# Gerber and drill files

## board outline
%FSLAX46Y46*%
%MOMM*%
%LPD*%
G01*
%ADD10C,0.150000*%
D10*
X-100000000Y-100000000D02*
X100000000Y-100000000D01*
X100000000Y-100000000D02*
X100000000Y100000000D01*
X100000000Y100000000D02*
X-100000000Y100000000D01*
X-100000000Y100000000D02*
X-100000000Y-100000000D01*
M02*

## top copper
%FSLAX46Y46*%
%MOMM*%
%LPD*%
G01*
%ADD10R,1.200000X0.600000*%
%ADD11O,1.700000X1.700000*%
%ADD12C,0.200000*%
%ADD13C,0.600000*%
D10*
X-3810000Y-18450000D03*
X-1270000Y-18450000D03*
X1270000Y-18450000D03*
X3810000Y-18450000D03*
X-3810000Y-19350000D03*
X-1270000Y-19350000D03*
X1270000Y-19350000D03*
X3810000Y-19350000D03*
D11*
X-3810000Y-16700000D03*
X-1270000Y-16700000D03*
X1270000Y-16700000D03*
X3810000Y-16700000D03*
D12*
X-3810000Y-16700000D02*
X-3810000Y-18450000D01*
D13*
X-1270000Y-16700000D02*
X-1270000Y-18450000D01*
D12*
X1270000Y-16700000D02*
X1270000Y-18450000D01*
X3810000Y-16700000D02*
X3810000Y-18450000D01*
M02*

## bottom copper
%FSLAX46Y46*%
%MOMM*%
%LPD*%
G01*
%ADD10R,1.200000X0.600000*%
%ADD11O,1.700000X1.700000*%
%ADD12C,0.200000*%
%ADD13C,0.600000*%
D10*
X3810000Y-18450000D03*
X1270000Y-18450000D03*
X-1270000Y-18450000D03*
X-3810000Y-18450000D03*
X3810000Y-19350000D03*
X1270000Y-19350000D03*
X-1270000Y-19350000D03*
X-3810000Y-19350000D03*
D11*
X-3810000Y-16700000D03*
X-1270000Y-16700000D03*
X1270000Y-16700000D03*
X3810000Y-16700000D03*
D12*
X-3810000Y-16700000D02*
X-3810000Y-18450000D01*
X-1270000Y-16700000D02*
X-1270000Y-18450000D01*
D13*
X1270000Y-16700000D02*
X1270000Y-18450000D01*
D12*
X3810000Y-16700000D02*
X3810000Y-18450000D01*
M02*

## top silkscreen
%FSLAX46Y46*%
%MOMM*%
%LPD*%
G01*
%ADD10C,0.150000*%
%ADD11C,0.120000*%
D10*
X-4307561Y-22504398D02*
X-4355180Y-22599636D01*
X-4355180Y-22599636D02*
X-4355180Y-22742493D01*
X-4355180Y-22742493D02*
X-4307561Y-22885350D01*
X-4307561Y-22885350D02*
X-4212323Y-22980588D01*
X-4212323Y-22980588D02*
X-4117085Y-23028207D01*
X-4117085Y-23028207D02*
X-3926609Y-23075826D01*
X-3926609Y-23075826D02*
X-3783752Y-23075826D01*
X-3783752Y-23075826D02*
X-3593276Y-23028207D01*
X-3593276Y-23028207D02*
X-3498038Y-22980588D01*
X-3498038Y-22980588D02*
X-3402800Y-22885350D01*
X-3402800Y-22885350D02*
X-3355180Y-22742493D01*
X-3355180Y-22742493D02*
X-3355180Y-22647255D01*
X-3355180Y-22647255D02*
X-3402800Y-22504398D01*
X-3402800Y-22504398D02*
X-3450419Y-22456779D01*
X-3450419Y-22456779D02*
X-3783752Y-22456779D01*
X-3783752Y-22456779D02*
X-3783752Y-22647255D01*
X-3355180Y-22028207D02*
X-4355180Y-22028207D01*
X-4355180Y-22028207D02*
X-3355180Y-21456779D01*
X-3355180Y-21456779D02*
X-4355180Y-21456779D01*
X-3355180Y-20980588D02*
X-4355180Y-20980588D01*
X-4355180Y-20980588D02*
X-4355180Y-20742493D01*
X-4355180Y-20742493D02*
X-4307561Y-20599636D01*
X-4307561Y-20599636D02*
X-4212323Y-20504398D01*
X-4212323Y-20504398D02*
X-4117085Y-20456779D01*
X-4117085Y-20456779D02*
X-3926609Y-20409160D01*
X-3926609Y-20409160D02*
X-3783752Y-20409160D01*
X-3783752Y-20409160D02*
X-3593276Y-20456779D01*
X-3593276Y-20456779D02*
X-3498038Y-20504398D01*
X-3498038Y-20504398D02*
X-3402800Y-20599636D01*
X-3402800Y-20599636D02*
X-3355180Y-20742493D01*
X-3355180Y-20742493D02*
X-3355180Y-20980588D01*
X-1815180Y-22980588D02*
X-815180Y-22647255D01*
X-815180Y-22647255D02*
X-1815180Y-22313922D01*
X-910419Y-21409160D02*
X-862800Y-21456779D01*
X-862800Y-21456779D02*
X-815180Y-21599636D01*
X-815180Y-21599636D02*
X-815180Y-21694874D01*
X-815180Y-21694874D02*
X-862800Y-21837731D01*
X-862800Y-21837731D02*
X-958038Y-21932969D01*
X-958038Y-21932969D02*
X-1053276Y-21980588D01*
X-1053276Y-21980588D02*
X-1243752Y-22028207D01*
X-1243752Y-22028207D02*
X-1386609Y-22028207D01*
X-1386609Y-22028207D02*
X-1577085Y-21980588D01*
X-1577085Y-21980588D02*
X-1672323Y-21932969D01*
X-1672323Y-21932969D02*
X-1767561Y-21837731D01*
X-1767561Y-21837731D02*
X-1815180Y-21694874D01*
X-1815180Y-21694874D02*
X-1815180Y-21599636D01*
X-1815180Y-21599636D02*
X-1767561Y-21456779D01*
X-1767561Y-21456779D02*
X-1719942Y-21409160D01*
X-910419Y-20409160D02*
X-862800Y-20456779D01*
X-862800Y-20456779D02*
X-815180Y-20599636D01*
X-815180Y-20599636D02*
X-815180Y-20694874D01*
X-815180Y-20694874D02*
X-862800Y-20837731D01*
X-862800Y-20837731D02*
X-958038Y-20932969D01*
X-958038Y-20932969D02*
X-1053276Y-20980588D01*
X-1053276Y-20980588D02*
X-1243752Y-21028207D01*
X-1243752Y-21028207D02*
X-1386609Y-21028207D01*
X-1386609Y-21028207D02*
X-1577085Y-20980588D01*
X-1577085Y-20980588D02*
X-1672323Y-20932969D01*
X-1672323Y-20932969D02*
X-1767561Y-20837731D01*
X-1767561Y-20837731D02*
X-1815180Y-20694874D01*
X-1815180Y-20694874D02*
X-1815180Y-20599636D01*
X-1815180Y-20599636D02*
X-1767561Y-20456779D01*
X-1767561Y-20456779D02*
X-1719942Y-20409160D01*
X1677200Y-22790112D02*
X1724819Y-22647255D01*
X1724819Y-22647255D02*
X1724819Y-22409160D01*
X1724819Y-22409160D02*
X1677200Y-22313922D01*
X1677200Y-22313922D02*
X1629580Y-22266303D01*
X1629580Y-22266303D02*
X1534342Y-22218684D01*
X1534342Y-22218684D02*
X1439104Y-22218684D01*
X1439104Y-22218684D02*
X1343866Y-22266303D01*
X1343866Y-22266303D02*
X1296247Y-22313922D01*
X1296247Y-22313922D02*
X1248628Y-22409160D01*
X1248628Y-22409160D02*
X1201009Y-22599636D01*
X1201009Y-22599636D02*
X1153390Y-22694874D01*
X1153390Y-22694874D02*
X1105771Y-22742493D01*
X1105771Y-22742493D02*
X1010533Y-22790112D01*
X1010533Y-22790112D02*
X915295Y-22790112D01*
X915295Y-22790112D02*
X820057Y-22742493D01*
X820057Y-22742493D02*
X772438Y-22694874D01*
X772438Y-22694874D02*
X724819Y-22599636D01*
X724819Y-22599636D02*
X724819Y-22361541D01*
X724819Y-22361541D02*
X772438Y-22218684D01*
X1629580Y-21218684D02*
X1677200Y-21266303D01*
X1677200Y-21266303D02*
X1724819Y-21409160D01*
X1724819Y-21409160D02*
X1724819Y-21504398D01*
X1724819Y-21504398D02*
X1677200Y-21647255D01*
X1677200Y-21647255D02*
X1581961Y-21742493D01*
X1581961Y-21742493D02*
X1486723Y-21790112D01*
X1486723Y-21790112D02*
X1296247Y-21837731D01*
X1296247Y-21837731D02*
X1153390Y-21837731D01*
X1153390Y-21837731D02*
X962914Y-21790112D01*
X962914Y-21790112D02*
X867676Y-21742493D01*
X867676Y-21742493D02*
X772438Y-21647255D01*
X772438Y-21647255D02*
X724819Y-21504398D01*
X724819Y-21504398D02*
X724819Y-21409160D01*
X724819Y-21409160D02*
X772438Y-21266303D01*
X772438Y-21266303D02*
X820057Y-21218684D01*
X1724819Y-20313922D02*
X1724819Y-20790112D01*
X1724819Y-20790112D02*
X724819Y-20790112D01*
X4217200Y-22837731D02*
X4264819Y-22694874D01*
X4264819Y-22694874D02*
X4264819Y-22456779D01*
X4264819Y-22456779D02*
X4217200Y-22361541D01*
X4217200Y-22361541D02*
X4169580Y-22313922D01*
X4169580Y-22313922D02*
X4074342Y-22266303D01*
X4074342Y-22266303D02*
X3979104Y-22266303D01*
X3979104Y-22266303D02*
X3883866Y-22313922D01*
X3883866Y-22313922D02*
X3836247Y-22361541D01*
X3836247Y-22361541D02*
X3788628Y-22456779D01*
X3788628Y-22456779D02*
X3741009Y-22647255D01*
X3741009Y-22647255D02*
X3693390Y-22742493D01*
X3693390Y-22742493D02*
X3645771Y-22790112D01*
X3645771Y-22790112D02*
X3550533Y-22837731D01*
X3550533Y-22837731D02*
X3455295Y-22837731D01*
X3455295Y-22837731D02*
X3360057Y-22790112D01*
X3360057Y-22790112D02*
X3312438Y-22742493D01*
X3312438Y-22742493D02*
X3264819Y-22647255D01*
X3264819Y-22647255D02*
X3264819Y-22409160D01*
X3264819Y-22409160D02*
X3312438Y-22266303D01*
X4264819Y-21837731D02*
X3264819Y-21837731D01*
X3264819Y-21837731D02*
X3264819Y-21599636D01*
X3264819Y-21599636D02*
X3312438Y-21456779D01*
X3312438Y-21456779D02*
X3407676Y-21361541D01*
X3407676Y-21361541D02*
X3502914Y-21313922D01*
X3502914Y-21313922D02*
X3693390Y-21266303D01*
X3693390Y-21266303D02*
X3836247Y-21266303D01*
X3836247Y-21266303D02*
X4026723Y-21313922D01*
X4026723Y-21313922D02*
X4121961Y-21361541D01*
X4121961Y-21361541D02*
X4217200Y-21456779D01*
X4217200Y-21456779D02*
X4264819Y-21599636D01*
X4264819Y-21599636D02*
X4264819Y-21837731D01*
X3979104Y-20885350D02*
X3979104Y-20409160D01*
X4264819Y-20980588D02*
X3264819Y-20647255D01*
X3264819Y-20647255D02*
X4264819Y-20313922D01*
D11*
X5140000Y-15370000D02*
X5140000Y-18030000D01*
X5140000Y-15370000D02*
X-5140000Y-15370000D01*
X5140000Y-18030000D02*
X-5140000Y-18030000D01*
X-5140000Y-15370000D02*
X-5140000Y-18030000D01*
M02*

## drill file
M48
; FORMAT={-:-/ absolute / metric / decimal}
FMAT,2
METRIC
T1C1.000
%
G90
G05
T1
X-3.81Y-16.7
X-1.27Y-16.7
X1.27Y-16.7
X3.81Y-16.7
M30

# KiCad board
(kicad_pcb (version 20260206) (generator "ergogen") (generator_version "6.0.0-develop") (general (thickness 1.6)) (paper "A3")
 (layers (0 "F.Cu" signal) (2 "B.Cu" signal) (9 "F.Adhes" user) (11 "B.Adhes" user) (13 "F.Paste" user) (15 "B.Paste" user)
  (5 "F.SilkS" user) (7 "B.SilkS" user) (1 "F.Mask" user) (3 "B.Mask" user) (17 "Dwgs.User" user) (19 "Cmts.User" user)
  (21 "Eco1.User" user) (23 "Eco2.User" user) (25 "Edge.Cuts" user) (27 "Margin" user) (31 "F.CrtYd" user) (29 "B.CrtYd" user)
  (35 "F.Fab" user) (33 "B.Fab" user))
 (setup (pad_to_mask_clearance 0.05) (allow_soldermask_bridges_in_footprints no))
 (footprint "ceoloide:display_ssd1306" (layer "F.Cu") (at 0 0 0)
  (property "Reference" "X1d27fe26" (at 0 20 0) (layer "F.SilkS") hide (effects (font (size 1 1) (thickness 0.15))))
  (fp_line (start 5.14 15.37) (end 5.14 18.03) (layer "F.SilkS") (stroke (width 0.12) (type solid)))
  (fp_line (start 5.14 15.37) (end -5.14 15.37) (layer "F.SilkS") (stroke (width 0.12) (type solid)))
  (fp_line (start 5.14 18.03) (end -5.14 18.03) (layer "F.SilkS") (stroke (width 0.12) (type solid)))
  (fp_line (start -5.14 15.37) (end -5.14 18.03) (layer "F.SilkS") (stroke (width 0.12) (type solid)))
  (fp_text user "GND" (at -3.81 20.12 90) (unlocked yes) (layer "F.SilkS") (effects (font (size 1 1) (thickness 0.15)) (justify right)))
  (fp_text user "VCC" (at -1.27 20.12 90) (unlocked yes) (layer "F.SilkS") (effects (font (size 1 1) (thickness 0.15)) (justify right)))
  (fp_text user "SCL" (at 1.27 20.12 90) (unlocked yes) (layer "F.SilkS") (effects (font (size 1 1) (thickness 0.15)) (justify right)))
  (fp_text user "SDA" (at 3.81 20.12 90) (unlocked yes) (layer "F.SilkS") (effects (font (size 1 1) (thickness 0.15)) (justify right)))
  (pad "14" smd rect (at -3.81 18.450000000000003 90) (size 0.6 1.2) (layers "F.Cu" "F.Paste" "F.Mask") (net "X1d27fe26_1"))
  (pad "15" smd rect (at -1.27 18.450000000000003 90) (size 0.6 1.2) (layers "F.Cu" "F.Paste" "F.Mask") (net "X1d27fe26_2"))
  (pad "16" smd rect (at 1.27 18.450000000000003 90) (size 0.6 1.2) (layers "F.Cu" "F.Paste" "F.Mask") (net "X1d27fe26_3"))
  (pad "17" smd rect (at 3.81 18.450000000000003 90) (size 0.6 1.2) (layers "F.Cu" "F.Paste" "F.Mask") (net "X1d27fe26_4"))
  (pad "10" smd rect (at -3.81 19.35 90) (size 0.6 1.2) (layers "F.Cu" "F.Paste" "F.Mask") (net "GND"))
  (pad "11" smd rect (at -1.27 19.35 90) (size 0.6 1.2) (layers "F.Cu" "F.Paste" "F.Mask") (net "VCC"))
  (pad "12" smd rect (at 1.27 19.35 90) (size 0.6 1.2) (layers "F.Cu" "F.Paste" "F.Mask") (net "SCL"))
  (pad "13" smd rect (at 3.81 19.35 90) (size 0.6 1.2) (layers "F.Cu" "F.Paste" "F.Mask") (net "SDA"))
  (pad "24" smd rect (at 3.81 18.450000000000003 270) (size 0.6 1.2) (layers "B.Cu" "B.Paste" "B.Mask") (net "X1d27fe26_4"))
  (pad "25" smd rect (at 1.27 18.450000000000003 270) (size 0.6 1.2) (layers "B.Cu" "B.Paste" "B.Mask") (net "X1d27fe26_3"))
  (pad "26" smd rect (at -1.27 18.450000000000003 270) (size 0.6 1.2) (layers "B.Cu" "B.Paste" "B.Mask") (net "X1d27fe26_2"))
  (pad "27" smd rect (at -3.81 18.450000000000003 270) (size 0.6 1.2) (layers "B.Cu" "B.Paste" "B.Mask") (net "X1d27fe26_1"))
  (pad "20" smd rect (at 3.81 19.35 270) (size 0.6 1.2) (layers "B.Cu" "B.Paste" "B.Mask") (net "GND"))
  (pad "21" smd rect (at 1.27 19.35 270) (size 0.6 1.2) (layers "B.Cu" "B.Paste" "B.Mask") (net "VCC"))
  (pad "22" smd rect (at -1.27 19.35 270) (size 0.6 1.2) (layers "B.Cu" "B.Paste" "B.Mask") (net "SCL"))
  (pad "23" smd rect (at -3.81 19.35 270) (size 0.6 1.2) (layers "B.Cu" "B.Paste" "B.Mask") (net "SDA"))
  (pad "1" thru_hole oval (at -3.81 16.7 270) (size 1.7 1.7) (drill 1) (layers "*.Cu" "*.Mask") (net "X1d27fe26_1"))
  (pad "2" thru_hole oval (at -1.27 16.7 270) (size 1.7 1.7) (drill 1) (layers "*.Cu" "*.Mask") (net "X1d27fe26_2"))
  (pad "3" thru_hole oval (at 1.27 16.7 270) (size 1.7 1.7) (drill 1) (layers "*.Cu" "*.Mask") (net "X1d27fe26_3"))
  (pad "4" thru_hole oval (at 3.81 16.7 270) (size 1.7 1.7) (drill 1) (layers "*.Cu" "*.Mask") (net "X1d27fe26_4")))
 (segment (start -3.81 16.7) (end -3.81 18.45) (width 0.2) (layer "F.Cu") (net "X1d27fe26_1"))
 (segment (start -1.27 16.7) (end -1.27 18.45) (width 0.6) (layer "F.Cu") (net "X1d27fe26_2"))
 (segment (start 1.27 16.7) (end 1.27 18.45) (width 0.2) (layer "F.Cu") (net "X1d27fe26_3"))
 (segment (start 3.81 16.7) (end 3.81 18.45) (width 0.2) (layer "F.Cu") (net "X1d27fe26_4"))
 (segment (start -3.81 16.7) (end -3.81 18.45) (width 0.2) (layer "B.Cu") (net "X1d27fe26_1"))
 (segment (start -1.27 16.7) (end -1.27 18.45) (width 0.2) (layer "B.Cu") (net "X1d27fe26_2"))
 (segment (start 1.27 16.7) (end 1.27 18.45) (width 0.6) (layer "B.Cu") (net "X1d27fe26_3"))
 (segment (start 3.81 16.7) (end 3.81 18.45) (width 0.2) (layer "B.Cu") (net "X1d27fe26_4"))
 (gr_line (start -100 100) (end 100 100) (layer Edge.Cuts) (stroke (width 0.15) (type default)))
 (gr_line (start 100 100) (end 100 -100) (layer Edge.Cuts) (stroke (width 0.15) (type default)))
 (gr_line (start 100 -100) (end -100 -100) (layer Edge.Cuts) (stroke (width 0.15) (type default)))
 (gr_line (start -100 -100) (end -100 100) (layer Edge.Cuts) (stroke (width 0.15) (type default))))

